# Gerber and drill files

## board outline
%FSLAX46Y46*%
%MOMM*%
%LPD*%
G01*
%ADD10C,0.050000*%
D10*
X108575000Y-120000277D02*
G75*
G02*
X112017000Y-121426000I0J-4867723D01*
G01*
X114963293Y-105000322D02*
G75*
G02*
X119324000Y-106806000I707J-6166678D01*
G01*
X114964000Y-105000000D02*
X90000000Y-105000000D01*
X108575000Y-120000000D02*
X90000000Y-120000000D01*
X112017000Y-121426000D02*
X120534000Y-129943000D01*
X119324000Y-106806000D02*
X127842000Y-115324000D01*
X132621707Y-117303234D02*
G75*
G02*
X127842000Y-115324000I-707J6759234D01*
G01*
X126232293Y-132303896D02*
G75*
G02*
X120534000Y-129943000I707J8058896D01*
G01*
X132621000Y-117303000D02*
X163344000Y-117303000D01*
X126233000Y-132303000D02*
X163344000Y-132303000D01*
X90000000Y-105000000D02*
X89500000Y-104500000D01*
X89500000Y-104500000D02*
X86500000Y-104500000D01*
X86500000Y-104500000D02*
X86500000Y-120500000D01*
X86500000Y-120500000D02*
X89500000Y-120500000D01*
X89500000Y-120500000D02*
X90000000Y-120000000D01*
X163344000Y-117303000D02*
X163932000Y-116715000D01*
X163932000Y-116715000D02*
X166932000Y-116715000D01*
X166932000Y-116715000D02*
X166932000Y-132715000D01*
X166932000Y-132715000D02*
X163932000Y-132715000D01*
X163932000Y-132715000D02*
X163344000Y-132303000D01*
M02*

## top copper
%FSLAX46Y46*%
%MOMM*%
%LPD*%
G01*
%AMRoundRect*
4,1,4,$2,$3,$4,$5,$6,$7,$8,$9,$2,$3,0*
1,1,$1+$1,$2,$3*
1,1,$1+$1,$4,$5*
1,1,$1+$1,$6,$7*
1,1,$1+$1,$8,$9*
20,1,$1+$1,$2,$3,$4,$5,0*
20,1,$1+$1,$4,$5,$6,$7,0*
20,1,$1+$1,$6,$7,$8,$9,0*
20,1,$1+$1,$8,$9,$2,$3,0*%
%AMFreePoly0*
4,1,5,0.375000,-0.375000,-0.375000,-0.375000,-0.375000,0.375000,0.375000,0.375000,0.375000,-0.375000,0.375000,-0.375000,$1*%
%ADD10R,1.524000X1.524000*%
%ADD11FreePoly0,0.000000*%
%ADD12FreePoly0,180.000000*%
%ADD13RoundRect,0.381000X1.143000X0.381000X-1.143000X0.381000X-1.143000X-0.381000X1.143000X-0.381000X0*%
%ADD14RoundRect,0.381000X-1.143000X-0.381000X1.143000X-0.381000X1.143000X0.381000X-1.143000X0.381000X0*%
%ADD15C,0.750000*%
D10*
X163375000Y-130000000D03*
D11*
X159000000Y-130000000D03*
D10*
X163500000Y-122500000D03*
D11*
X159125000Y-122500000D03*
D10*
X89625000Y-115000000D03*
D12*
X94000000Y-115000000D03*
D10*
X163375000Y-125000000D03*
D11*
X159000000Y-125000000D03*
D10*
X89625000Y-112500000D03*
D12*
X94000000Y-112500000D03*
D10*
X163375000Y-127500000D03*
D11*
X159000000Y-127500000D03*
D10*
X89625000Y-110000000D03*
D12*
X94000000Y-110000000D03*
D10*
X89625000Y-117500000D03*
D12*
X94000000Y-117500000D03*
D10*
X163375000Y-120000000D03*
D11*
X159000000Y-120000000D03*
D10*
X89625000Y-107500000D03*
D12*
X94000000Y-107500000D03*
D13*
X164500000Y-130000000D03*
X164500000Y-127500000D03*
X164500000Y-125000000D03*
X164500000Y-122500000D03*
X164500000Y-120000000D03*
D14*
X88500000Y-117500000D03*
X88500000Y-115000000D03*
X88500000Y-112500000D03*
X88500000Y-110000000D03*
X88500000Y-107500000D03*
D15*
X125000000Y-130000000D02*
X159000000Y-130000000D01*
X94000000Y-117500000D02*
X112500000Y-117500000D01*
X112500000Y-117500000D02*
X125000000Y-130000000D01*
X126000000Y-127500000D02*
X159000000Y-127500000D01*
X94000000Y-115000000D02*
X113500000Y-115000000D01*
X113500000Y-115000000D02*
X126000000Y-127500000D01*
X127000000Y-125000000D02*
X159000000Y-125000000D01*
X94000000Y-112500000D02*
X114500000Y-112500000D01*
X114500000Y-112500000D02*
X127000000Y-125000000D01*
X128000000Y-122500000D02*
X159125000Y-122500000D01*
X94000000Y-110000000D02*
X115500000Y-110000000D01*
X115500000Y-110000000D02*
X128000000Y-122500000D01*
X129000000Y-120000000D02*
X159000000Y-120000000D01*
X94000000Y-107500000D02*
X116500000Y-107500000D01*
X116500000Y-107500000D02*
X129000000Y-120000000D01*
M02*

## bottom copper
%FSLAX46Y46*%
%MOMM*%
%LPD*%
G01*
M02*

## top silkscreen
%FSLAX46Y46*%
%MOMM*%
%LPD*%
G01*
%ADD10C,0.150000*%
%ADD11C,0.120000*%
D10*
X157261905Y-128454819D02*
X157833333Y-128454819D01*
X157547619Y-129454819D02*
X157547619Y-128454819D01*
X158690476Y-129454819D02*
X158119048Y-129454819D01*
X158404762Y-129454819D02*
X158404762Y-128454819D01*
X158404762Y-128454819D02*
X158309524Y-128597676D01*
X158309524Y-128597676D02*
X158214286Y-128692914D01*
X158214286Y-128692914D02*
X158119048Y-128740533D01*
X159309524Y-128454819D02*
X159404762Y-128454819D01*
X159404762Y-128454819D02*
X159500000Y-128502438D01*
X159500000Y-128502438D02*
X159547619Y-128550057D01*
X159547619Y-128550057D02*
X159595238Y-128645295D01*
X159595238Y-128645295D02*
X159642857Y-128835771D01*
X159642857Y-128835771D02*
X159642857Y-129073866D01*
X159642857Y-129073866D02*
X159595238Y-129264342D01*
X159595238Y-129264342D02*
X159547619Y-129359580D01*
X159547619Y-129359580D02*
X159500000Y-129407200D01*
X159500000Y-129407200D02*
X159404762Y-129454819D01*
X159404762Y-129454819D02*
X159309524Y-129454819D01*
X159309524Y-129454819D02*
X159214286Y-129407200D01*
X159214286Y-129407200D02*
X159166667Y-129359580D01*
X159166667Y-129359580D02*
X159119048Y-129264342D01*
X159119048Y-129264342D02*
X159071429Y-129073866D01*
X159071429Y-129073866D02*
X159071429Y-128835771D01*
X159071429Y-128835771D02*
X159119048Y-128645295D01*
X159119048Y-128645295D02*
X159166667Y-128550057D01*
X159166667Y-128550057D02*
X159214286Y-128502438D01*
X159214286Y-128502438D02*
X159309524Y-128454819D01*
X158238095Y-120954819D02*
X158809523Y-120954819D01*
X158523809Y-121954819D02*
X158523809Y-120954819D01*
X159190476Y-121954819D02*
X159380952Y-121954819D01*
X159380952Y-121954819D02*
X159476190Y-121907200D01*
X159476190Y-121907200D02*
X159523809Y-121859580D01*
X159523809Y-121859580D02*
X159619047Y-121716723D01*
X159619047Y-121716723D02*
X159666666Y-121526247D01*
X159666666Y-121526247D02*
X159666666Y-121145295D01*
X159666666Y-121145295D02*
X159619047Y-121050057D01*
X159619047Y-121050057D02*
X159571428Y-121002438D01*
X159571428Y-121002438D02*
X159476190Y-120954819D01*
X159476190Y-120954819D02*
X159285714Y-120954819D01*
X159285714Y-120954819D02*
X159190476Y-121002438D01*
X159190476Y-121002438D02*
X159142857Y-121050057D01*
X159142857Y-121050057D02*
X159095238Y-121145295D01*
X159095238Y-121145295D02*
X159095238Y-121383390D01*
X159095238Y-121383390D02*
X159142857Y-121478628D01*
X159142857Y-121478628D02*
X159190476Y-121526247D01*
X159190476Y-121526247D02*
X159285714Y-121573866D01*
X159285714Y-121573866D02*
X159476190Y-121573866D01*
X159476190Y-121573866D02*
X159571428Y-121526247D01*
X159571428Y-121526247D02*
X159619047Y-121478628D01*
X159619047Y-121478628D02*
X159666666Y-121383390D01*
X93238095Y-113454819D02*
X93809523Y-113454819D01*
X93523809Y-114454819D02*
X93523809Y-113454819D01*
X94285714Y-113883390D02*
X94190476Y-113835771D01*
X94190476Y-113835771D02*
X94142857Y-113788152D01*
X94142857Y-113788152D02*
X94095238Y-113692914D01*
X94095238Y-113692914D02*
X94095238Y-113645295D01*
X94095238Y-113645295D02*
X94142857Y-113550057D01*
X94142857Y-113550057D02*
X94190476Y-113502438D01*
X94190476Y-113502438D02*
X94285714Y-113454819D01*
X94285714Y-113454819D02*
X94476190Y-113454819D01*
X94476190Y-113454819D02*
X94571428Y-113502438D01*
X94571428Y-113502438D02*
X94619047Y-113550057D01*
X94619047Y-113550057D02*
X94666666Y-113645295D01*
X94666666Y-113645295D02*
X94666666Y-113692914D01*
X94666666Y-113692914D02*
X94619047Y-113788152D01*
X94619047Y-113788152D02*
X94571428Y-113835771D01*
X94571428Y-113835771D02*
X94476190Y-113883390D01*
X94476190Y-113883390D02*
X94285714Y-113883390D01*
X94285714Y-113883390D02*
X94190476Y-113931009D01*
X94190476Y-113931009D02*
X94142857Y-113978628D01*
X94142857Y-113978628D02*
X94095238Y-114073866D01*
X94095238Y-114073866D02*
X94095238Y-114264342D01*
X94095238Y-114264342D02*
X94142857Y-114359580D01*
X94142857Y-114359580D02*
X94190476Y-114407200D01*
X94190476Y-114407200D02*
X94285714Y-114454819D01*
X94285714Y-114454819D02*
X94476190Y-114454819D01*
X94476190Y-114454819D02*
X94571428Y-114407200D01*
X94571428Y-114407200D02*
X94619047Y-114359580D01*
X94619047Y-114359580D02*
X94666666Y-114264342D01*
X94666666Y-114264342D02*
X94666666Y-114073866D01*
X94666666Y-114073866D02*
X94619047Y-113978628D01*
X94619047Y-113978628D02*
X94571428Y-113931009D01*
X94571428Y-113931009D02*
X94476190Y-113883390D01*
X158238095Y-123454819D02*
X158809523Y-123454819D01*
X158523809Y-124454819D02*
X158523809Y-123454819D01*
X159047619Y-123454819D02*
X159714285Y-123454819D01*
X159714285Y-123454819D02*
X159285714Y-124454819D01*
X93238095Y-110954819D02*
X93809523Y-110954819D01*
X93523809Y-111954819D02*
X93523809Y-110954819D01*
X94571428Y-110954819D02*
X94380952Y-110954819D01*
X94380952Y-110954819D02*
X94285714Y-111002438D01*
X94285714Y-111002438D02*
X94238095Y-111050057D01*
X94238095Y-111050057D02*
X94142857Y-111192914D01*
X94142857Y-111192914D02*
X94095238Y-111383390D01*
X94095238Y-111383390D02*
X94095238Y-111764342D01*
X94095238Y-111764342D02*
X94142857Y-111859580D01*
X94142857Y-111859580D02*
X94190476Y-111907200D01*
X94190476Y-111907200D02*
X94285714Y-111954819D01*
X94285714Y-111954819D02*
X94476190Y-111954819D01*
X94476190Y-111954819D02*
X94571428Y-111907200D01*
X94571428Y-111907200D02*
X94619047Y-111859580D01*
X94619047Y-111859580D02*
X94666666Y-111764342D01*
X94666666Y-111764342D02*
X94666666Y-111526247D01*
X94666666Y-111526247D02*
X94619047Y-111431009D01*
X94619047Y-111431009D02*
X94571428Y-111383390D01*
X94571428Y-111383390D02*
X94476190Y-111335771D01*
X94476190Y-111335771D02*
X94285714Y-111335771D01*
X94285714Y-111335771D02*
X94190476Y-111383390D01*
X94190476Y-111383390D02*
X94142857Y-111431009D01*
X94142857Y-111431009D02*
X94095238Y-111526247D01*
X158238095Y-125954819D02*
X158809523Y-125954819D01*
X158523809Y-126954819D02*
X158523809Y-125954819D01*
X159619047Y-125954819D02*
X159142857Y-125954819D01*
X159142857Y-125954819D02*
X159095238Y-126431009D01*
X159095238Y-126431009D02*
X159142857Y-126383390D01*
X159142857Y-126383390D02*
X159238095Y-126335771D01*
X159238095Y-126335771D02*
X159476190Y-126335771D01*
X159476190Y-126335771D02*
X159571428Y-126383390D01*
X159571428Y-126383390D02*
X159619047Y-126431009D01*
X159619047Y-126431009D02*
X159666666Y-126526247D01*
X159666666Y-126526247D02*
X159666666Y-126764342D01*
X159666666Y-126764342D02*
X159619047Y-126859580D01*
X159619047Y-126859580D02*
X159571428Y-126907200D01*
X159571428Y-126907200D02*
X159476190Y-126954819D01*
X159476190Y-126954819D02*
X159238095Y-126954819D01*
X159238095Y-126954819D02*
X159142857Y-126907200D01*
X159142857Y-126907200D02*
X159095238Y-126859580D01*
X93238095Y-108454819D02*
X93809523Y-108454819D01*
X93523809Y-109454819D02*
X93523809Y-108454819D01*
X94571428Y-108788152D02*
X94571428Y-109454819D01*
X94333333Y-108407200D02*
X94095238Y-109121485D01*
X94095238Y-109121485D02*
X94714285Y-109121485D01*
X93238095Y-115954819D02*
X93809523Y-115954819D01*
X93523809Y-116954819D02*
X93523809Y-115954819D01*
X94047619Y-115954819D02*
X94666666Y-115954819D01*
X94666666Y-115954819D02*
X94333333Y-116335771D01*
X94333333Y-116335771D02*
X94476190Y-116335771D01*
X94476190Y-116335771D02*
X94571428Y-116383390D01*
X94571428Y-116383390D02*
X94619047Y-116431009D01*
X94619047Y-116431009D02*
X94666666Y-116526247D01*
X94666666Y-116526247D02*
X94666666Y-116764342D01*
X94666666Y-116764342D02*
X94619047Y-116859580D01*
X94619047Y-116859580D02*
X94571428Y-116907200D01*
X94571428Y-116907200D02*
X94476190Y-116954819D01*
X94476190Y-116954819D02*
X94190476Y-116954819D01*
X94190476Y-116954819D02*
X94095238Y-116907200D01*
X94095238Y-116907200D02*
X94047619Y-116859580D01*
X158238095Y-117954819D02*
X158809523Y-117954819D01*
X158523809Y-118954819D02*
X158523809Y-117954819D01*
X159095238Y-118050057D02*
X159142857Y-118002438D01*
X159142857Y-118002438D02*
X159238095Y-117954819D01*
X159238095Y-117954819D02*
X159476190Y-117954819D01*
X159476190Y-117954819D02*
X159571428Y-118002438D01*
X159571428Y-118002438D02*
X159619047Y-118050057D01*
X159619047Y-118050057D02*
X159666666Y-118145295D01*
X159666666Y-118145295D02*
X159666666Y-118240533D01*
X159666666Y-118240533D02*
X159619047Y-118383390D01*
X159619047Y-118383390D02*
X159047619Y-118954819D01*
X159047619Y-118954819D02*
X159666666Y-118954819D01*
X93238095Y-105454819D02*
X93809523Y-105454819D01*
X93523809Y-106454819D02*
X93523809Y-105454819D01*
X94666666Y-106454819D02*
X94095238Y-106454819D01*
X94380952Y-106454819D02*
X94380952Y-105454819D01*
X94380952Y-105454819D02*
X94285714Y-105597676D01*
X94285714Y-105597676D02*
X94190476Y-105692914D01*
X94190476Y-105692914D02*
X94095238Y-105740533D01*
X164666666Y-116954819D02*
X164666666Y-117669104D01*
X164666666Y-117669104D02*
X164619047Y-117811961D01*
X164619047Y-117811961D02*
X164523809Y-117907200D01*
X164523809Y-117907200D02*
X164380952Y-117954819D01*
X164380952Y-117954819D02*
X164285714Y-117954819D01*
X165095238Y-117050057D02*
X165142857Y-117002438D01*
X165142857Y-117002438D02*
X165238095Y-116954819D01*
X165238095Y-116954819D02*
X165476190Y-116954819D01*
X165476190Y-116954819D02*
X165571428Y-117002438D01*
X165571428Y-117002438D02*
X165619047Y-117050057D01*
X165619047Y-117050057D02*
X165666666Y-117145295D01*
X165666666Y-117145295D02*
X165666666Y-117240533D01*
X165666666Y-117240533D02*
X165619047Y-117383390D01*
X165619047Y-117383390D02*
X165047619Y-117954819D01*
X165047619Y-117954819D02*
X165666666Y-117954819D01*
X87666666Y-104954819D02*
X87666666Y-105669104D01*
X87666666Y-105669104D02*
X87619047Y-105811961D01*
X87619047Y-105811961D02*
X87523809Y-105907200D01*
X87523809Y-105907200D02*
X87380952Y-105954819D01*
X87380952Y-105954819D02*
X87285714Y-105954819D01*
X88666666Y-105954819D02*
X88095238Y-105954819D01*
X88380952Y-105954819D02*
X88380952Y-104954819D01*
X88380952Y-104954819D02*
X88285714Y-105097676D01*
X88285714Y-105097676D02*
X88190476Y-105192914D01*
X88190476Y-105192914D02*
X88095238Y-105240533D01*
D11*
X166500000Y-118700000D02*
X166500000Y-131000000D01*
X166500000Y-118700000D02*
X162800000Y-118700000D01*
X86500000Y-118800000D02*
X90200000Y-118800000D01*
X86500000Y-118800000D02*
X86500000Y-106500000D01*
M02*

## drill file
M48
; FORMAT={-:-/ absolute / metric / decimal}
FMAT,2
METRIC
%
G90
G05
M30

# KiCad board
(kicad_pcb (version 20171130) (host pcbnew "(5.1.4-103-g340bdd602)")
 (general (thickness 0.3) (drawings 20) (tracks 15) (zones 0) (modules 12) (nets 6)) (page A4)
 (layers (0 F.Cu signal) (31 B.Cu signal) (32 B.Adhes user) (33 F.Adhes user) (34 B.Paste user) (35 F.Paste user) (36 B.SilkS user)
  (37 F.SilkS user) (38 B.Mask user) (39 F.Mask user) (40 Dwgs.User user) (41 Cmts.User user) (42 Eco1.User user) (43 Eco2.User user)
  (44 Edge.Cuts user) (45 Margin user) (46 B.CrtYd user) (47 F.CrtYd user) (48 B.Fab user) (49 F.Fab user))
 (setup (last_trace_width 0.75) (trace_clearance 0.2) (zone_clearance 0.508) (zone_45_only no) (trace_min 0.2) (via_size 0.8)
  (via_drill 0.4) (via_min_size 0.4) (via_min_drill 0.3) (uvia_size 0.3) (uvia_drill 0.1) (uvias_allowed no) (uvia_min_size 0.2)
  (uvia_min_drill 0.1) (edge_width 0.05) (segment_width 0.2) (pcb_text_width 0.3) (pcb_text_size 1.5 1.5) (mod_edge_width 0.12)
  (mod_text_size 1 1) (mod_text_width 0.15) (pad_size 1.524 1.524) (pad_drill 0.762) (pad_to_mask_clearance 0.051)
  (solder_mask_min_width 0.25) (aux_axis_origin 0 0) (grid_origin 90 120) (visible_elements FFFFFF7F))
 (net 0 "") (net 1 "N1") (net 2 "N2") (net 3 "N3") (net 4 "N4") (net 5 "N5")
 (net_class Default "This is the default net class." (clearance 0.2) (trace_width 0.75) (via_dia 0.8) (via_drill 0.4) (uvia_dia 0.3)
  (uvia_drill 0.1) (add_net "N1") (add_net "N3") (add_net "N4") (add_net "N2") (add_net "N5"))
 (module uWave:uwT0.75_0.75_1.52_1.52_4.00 (layer F.Cu) (at 159 130)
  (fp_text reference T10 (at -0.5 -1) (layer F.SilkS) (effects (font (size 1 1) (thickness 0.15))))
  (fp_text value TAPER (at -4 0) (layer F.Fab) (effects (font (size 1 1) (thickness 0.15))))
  (pad 1 smd rect (at 4.375 0) (size 1.524 1.524) (layers F.Cu) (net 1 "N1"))
  (pad 1 smd custom (at 0 0) (size 0.75 0.75) (layers F.Cu) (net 1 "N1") (options (clearance outline) (anchor rect)) (primitives)))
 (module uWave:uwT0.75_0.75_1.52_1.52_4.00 (layer F.Cu) (at 159.125 122.5)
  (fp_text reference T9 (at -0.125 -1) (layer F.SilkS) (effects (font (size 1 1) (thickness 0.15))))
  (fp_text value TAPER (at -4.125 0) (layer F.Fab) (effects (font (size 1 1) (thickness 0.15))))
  (pad 1 smd rect (at 4.375 0) (size 1.524 1.524) (layers F.Cu) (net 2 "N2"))
  (pad 1 smd custom (at 0 0) (size 0.75 0.75) (layers F.Cu) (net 2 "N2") (options (clearance outline) (anchor rect)) (primitives)))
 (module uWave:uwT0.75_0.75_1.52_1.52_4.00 (layer F.Cu) (at 94 115 180)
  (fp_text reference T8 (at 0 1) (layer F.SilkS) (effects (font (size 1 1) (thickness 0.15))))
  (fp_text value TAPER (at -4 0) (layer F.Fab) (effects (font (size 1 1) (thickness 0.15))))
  (pad 1 smd rect (at 4.375 0 180) (size 1.524 1.524) (layers F.Cu) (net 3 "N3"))
  (pad 1 smd custom (at 0 0 180) (size 0.75 0.75) (layers F.Cu) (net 3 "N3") (options (clearance outline) (anchor rect)) (primitives)))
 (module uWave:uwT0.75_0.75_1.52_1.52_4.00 (layer F.Cu) (at 159 125)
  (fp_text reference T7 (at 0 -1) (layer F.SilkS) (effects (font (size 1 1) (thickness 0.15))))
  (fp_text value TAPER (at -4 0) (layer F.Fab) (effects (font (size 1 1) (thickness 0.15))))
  (pad 1 smd rect (at 4.375 0) (size 1.524 1.524) (layers F.Cu) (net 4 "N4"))
  (pad 1 smd custom (at 0 0) (size 0.75 0.75) (layers F.Cu) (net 4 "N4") (options (clearance outline) (anchor rect)) (primitives)))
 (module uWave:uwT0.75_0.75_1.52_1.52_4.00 (layer F.Cu) (at 94 112.5 180)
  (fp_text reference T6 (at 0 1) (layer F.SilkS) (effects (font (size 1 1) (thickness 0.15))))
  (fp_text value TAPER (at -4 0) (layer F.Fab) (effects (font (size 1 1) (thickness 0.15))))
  (pad 1 smd rect (at 4.375 0 180) (size 1.524 1.524) (layers F.Cu) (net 4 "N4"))
  (pad 1 smd custom (at 0 0 180) (size 0.75 0.75) (layers F.Cu) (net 4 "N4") (options (clearance outline) (anchor rect)) (primitives)))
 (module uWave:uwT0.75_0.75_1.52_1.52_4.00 (layer F.Cu) (at 159 127.5)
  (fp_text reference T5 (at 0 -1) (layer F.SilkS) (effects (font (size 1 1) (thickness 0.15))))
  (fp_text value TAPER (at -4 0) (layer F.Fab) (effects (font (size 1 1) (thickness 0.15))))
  (pad 1 smd rect (at 4.375 0) (size 1.524 1.524) (layers F.Cu) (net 3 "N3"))
  (pad 1 smd custom (at 0 0) (size 0.75 0.75) (layers F.Cu) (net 3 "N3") (options (clearance outline) (anchor rect)) (primitives)))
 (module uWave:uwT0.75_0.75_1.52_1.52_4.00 (layer F.Cu) (at 94 110 180)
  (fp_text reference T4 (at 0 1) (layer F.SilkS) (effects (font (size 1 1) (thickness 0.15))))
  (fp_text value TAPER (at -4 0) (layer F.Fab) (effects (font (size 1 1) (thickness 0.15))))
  (pad 1 smd rect (at 4.375 0 180) (size 1.524 1.524) (layers F.Cu) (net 2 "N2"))
  (pad 1 smd custom (at 0 0 180) (size 0.75 0.75) (layers F.Cu) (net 2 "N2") (options (clearance outline) (anchor rect)) (primitives)))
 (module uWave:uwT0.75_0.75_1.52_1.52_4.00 (layer F.Cu) (at 94 117.5 180)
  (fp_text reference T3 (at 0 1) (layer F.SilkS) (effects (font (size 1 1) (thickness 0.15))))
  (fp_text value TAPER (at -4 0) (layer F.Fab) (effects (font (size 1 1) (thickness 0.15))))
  (pad 1 smd rect (at 4.375 0 180) (size 1.524 1.524) (layers F.Cu) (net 1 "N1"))
  (pad 1 smd custom (at 0 0 180) (size 0.75 0.75) (layers F.Cu) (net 1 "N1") (options (clearance outline) (anchor rect)) (primitives)))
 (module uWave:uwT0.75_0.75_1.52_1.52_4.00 (layer F.Cu) (at 159 120)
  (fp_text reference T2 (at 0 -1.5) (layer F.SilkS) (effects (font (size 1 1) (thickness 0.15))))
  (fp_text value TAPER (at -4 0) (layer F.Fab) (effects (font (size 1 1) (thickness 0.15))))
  (pad 1 smd rect (at 4.375 0) (size 1.524 1.524) (layers F.Cu) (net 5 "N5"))
  (pad 1 smd custom (at 0 0) (size 0.75 0.75) (layers F.Cu) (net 5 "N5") (options (clearance outline) (anchor rect)) (primitives)))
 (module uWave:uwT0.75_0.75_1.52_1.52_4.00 (layer F.Cu) (at 94 107.5 180)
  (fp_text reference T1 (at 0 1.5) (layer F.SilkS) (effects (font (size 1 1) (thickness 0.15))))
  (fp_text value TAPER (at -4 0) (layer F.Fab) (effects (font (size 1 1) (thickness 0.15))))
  (pad 1 smd rect (at 4.375 0 180) (size 1.524 1.524) (layers F.Cu) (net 5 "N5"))
  (pad 1 smd custom (at 0 0 180) (size 0.75 0.75) (layers F.Cu) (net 5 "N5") (options (clearance outline) (anchor rect)) (primitives)))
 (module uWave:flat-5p (layer F.Cu) (at 164.5 120 180)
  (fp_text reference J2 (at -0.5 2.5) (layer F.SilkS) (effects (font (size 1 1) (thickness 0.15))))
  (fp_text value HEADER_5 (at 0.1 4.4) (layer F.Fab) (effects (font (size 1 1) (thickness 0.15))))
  (fp_line (start -2 1.3) (end -2 -11) (layer F.SilkS) (width 0.12))
  (fp_line (start -2 1.3) (end 1.7 1.3) (layer F.SilkS) (width 0.12))
  (pad 5 smd roundrect (at 0 -10 180) (size 3.048 1.524) (layers F.Cu F.Paste F.Mask) (roundrect_rratio 0.25) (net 1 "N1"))
  (pad 4 smd roundrect (at 0 -7.5 180) (size 3.048 1.524) (layers F.Cu F.Paste F.Mask) (roundrect_rratio 0.25) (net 3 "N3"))
  (pad 3 smd roundrect (at 0 -5 180) (size 3.048 1.524) (layers F.Cu F.Paste F.Mask) (roundrect_rratio 0.25) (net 4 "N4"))
  (pad 2 smd roundrect (at 0 -2.5 180) (size 3.048 1.524) (layers F.Cu F.Paste F.Mask) (roundrect_rratio 0.25) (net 2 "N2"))
  (pad 1 smd roundrect (at 0 0 180) (size 3.048 1.524) (layers F.Cu F.Paste F.Mask) (roundrect_rratio 0.25) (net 5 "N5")))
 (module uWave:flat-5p (layer F.Cu) (at 88.5 117.5)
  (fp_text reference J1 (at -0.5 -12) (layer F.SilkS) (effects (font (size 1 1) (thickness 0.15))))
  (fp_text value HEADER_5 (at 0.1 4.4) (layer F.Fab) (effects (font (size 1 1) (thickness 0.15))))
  (fp_line (start -2 1.3) (end 1.7 1.3) (layer F.SilkS) (width 0.12))
  (fp_line (start -2 1.3) (end -2 -11) (layer F.SilkS) (width 0.12))
  (pad 1 smd roundrect (at 0 0) (size 3.048 1.524) (layers F.Cu F.Paste F.Mask) (roundrect_rratio 0.25) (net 1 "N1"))
  (pad 2 smd roundrect (at 0 -2.5) (size 3.048 1.524) (layers F.Cu F.Paste F.Mask) (roundrect_rratio 0.25) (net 3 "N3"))
  (pad 3 smd roundrect (at 0 -5) (size 3.048 1.524) (layers F.Cu F.Paste F.Mask) (roundrect_rratio 0.25) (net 4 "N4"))
  (pad 4 smd roundrect (at 0 -7.5) (size 3.048 1.524) (layers F.Cu F.Paste F.Mask) (roundrect_rratio 0.25) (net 2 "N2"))
  (pad 5 smd roundrect (at 0 -10) (size 3.048 1.524) (layers F.Cu F.Paste F.Mask) (roundrect_rratio 0.25) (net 5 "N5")))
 (gr_arc (start 108.575 124.868) (end 112.017 121.426) (angle -45) (layer Edge.Cuts) (width 0.05))
 (gr_arc (start 114.964 111.167) (end 119.324 106.806) (angle -45) (layer Edge.Cuts) (width 0.05))
 (gr_line (start 114.964 105) (end 90 105) (angle 90) (layer Edge.Cuts) (width 0.05))
 (gr_line (start 108.575 120) (end 90 120) (angle 90) (layer Edge.Cuts) (width 0.05))
 (gr_line (start 112.017 121.426) (end 120.534 129.943) (angle 90) (layer Edge.Cuts) (width 0.05))
 (gr_line (start 119.324 106.806) (end 127.842 115.324) (angle 90) (layer Edge.Cuts) (width 0.05))
 (gr_arc (start 132.621 110.544) (end 127.842 115.324) (angle -45) (layer Edge.Cuts) (width 0.05))
 (gr_arc (start 126.233 124.245) (end 120.534 129.943) (angle -45) (layer Edge.Cuts) (width 0.05))
 (gr_line (start 132.621 117.303) (end 163.344 117.303) (angle 90) (layer Edge.Cuts) (width 0.05))
 (gr_line (start 126.233 132.303) (end 163.344 132.303) (angle 90) (layer Edge.Cuts) (width 0.05))
 (gr_line (start 90 105) (end 89.5 104.5) (angle 90) (layer Edge.Cuts) (width 0.05))
 (gr_line (start 89.5 104.5) (end 86.5 104.5) (angle 90) (layer Edge.Cuts) (width 0.05))
 (gr_line (start 86.5 104.5) (end 86.5 120.5) (angle 90) (layer Edge.Cuts) (width 0.05))
 (gr_line (start 86.5 120.5) (end 89.5 120.5) (angle 90) (layer Edge.Cuts) (width 0.05))
 (gr_line (start 89.5 120.5) (end 90 120) (angle 90) (layer Edge.Cuts) (width 0.05))
 (gr_line (start 163.344 117.303) (end 163.932 116.715) (angle 90) (layer Edge.Cuts) (width 0.05))
 (gr_line (start 163.932 116.715) (end 166.932 116.715) (angle 90) (layer Edge.Cuts) (width 0.05))
 (gr_line (start 166.932 116.715) (end 166.932 132.715) (angle 90) (layer Edge.Cuts) (width 0.05))
 (gr_line (start 166.932 132.715) (end 163.932 132.715) (angle 90) (layer Edge.Cuts) (width 0.05))
 (gr_line (start 163.932 132.715) (end 163.344 132.303) (angle 90) (layer Edge.Cuts) (width 0.05))
 (segment (start 125 130) (end 159 130) (width 0.75) (layer F.Cu) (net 1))
 (segment (start 94 117.5) (end 112.5 117.5) (width 0.75) (layer F.Cu) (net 1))
 (segment (start 112.5 117.5) (end 125 130) (width 0.75) (layer F.Cu) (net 1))
 (segment (start 126 127.5) (end 159 127.5) (width 0.75) (layer F.Cu) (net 3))
 (segment (start 94 115) (end 113.5 115) (width 0.75) (layer F.Cu) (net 3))
 (segment (start 113.5 115) (end 126 127.5) (width 0.75) (layer F.Cu) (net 3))
 (segment (start 127 125) (end 159 125) (width 0.75) (layer F.Cu) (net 4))
 (segment (start 94 112.5) (end 114.5 112.5) (width 0.75) (layer F.Cu) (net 4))
 (segment (start 114.5 112.5) (end 127 125) (width 0.75) (layer F.Cu) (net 4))
 (segment (start 128 122.5) (end 159.125 122.5) (width 0.75) (layer F.Cu) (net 2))
 (segment (start 94 110) (end 115.5 110) (width 0.75) (layer F.Cu) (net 2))
 (segment (start 115.5 110) (end 128 122.5) (width 0.75) (layer F.Cu) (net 2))
 (segment (start 129 120) (end 159 120) (width 0.75) (layer F.Cu) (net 5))
 (segment (start 94 107.5) (end 116.5 107.5) (width 0.75) (layer F.Cu) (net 5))
 (segment (start 116.5 107.5) (end 129 120) (width 0.75) (layer F.Cu) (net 5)))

